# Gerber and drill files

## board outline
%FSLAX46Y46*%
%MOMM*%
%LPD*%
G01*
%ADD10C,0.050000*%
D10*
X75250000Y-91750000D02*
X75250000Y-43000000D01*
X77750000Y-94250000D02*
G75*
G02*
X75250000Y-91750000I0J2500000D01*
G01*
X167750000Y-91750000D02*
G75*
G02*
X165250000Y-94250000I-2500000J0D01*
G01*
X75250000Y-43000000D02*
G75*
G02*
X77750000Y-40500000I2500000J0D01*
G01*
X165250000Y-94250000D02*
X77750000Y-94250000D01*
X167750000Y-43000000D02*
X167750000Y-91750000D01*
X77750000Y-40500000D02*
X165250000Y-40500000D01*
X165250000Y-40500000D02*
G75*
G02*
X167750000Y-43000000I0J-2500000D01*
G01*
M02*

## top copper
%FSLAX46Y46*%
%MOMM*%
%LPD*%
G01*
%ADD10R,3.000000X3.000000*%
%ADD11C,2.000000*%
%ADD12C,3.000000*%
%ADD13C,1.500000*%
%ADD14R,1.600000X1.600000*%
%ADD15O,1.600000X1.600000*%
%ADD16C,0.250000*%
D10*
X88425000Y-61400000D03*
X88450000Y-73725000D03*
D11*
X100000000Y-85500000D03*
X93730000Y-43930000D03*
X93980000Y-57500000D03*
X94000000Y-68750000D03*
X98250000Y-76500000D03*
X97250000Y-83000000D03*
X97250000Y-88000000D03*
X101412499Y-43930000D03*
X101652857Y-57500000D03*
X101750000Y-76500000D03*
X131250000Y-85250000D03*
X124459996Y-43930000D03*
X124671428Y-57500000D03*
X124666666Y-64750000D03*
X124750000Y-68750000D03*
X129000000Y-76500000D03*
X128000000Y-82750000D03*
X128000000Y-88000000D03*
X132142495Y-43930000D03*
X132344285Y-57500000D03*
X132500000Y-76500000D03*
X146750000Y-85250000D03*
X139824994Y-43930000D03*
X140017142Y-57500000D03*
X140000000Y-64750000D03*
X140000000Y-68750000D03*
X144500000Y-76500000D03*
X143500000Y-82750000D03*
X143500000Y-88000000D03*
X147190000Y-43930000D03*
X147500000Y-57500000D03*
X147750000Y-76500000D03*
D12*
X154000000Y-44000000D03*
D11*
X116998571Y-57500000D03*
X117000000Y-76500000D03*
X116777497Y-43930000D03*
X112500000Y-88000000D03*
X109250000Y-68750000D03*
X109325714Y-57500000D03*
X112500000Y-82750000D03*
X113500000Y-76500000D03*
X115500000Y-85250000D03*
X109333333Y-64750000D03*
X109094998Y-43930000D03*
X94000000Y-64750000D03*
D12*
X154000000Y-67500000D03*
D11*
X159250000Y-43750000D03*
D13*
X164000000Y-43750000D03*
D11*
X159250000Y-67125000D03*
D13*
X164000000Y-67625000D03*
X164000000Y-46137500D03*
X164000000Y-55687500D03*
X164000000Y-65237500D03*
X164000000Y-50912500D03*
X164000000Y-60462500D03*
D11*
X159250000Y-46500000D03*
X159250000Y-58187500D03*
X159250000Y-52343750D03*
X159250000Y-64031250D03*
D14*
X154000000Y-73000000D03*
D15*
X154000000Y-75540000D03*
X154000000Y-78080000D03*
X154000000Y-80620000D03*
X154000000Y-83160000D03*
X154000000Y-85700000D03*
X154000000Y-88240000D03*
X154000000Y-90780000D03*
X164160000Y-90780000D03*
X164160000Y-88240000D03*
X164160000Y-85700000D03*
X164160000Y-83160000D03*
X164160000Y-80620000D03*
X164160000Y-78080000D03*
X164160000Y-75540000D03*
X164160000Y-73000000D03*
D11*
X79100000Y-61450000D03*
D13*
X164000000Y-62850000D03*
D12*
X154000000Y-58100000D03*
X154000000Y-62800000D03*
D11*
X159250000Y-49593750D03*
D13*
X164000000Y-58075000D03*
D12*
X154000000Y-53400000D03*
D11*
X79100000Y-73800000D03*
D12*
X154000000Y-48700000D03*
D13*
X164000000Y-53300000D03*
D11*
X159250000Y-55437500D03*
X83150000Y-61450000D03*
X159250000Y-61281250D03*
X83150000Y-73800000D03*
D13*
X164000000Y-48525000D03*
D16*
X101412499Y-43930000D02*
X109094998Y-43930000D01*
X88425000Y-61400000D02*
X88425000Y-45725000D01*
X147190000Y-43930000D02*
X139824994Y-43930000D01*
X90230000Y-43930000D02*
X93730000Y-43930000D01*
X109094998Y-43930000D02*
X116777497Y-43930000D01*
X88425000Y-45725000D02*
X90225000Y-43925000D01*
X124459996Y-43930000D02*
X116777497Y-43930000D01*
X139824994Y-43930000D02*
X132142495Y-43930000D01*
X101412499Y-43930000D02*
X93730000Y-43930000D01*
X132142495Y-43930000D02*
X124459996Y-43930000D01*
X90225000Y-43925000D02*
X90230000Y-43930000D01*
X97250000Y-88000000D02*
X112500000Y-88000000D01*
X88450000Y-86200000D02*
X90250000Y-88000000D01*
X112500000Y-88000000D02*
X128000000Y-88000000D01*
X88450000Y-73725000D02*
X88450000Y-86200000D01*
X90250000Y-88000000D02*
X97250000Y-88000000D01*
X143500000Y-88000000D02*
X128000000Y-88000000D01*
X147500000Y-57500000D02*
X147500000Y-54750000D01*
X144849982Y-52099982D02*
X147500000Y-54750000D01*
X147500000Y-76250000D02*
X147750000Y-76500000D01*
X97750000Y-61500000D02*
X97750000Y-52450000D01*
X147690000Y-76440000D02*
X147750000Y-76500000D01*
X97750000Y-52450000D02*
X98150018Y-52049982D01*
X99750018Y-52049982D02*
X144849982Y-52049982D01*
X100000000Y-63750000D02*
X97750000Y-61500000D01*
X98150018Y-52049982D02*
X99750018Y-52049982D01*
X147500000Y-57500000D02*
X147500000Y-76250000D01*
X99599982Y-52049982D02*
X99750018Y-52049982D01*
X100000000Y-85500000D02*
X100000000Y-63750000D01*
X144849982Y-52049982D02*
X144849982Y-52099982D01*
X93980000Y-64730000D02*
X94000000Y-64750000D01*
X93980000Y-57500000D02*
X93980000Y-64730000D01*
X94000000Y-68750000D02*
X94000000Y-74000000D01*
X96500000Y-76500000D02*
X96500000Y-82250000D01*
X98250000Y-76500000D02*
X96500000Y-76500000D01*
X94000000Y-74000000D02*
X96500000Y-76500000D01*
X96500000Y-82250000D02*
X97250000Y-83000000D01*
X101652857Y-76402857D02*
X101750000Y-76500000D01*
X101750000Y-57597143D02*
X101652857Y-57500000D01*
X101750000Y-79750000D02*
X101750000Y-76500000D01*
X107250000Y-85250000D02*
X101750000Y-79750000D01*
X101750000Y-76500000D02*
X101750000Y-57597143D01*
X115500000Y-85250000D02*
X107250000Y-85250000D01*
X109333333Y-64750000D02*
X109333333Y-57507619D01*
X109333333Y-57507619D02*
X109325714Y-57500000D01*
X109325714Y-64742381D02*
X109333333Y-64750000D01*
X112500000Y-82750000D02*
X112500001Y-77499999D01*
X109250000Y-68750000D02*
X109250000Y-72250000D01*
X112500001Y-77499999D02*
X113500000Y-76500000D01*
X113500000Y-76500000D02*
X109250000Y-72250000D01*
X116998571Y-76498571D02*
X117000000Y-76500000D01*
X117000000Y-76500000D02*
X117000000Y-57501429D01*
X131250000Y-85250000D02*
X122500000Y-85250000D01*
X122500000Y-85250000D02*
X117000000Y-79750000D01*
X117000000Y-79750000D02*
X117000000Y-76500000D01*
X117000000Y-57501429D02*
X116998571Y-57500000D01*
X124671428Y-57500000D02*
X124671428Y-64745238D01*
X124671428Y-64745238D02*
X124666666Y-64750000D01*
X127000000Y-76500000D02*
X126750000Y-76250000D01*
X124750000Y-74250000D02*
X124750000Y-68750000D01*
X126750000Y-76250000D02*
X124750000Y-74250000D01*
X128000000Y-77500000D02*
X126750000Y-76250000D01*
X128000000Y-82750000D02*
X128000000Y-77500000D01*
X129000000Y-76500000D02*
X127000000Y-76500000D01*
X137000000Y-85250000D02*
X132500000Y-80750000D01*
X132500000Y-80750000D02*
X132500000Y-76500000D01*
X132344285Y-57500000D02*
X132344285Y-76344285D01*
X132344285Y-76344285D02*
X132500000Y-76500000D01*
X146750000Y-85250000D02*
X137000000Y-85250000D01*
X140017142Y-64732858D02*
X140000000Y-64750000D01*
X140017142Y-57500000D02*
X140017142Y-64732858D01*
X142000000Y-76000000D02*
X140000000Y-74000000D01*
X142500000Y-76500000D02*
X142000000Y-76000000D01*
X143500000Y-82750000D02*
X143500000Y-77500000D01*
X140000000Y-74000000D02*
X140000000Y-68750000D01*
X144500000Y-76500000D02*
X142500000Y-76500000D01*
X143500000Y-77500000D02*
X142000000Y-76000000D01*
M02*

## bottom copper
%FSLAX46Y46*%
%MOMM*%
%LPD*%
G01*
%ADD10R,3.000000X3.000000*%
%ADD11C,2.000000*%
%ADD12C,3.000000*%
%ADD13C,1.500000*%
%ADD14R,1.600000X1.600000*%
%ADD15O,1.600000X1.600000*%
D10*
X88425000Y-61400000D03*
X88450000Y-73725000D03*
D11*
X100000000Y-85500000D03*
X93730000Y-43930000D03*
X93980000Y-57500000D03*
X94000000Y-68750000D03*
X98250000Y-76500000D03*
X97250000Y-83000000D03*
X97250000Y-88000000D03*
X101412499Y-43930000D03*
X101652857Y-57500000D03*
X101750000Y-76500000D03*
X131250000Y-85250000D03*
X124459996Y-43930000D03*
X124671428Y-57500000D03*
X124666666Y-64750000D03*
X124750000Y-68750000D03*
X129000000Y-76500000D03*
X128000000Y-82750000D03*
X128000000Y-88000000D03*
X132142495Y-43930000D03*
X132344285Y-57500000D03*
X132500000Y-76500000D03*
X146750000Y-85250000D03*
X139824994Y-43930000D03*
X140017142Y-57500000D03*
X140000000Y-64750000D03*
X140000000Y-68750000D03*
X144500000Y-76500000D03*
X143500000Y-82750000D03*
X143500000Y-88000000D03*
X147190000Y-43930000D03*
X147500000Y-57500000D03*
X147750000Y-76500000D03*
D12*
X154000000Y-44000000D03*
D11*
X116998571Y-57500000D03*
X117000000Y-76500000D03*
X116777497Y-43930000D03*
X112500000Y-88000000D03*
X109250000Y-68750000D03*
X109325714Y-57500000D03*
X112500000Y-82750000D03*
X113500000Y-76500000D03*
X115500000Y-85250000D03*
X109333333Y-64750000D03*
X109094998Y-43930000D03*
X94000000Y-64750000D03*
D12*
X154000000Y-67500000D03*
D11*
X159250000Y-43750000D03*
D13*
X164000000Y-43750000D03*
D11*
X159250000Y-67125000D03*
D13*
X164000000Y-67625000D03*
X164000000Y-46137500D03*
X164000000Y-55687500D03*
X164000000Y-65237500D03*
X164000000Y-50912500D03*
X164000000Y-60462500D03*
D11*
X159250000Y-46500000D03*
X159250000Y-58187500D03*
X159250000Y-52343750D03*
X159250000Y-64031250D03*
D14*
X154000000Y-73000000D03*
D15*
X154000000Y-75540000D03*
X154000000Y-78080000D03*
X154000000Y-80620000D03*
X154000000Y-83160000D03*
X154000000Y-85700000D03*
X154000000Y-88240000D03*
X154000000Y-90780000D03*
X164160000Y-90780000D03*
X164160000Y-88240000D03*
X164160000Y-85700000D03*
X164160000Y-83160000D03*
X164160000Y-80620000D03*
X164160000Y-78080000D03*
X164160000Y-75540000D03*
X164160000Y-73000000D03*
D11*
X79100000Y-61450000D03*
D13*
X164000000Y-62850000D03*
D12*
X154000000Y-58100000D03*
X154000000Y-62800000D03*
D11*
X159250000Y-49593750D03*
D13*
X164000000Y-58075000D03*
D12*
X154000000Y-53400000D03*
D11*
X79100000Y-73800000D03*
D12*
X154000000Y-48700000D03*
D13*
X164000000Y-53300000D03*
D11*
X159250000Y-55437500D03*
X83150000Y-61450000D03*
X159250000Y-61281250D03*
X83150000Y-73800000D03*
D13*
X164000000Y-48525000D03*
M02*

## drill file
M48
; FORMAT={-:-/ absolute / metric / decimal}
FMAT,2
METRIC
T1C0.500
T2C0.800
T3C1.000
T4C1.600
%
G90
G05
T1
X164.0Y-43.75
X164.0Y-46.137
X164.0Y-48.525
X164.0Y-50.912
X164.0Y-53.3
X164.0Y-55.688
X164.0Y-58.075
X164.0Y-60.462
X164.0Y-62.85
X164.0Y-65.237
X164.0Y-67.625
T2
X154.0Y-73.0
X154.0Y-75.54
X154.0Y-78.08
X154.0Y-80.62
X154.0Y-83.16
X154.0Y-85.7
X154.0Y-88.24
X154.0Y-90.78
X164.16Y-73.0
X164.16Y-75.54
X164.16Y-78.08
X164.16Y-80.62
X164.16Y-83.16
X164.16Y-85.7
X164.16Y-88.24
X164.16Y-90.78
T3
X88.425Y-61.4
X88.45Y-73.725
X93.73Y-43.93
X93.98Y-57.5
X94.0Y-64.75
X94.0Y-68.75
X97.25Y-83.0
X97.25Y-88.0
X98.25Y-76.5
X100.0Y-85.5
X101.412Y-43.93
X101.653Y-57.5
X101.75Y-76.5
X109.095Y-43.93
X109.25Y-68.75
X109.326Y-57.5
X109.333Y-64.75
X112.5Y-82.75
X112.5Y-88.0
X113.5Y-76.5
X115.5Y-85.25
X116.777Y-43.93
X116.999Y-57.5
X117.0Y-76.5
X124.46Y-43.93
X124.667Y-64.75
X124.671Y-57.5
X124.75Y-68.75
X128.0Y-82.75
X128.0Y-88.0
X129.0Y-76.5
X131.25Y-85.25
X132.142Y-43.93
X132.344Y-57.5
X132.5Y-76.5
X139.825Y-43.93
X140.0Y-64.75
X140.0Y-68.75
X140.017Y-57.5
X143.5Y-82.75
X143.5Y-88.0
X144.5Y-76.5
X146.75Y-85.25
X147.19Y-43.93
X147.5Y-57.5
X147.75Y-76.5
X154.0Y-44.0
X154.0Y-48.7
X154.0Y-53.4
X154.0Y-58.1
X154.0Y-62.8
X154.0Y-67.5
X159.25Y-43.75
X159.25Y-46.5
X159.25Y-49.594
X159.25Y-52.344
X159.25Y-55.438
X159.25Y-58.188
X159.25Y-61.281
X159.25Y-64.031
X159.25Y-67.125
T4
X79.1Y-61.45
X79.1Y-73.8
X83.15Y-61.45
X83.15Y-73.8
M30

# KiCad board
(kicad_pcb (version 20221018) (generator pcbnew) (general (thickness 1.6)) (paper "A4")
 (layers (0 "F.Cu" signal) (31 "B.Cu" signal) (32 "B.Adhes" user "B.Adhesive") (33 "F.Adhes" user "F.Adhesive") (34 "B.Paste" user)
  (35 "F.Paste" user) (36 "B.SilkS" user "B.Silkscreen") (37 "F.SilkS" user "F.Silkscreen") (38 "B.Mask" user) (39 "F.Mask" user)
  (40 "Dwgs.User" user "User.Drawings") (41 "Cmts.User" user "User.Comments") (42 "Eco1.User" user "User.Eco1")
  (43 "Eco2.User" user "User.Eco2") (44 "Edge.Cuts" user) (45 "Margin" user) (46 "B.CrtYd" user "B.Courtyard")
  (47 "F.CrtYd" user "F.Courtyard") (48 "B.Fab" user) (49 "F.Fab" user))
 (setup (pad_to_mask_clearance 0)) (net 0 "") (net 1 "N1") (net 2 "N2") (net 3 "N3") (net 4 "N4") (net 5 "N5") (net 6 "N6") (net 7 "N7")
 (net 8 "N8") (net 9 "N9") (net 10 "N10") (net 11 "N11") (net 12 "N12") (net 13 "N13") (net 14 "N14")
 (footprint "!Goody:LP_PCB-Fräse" (layer "F.Cu") (at 88.425 61.4)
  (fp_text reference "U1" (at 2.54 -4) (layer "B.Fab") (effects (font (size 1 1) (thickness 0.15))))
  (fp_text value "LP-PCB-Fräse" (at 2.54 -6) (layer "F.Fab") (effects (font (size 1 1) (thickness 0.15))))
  (pad "1" thru_hole rect (at 0 0) (size 3 3) (drill 1) (layers "*.Cu" "*.Mask") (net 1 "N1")))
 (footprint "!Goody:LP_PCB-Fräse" (layer "F.Cu") (at 88.45 73.725)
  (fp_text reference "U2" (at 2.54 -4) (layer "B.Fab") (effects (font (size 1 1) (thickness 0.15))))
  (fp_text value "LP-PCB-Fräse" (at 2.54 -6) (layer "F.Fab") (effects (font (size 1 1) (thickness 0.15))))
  (pad "1" thru_hole rect (at 0 0) (size 3 3) (drill 1) (layers "*.Cu" "*.Mask") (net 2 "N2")))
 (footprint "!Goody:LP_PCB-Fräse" (layer "F.Cu") (at 100 85.5)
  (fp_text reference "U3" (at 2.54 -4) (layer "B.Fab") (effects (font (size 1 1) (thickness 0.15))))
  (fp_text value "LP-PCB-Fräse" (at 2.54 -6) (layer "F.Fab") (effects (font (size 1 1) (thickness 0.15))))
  (pad "1" thru_hole circle (at 0 0) (size 2 2) (drill 1) (layers "*.Cu" "*.Mask") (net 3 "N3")))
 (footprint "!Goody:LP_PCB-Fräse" (layer "F.Cu") (at 93.73 43.93)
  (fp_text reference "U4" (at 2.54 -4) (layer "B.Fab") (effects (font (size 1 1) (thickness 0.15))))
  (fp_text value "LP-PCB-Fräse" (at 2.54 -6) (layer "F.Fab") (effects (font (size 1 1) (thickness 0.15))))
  (pad "1" thru_hole circle (at 0 0) (size 2 2) (drill 1) (layers "*.Cu" "*.Mask") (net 1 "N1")))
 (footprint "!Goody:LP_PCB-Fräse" (layer "F.Cu") (at 93.98 57.5)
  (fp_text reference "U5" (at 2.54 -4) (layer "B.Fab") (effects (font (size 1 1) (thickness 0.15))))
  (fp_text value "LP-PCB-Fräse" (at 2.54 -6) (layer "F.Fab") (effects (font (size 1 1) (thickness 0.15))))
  (pad "1" thru_hole circle (at 0 0) (size 2 2) (drill 1) (layers "*.Cu" "*.Mask") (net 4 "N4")))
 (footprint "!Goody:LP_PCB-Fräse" (layer "F.Cu") (at 94 68.75)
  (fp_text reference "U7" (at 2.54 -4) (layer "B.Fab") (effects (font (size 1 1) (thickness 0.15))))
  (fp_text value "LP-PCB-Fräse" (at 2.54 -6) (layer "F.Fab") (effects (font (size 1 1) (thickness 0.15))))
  (pad "1" thru_hole circle (at 0 0) (size 2 2) (drill 1) (layers "*.Cu" "*.Mask") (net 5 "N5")))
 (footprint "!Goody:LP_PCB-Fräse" (layer "F.Cu") (at 98.25 76.5)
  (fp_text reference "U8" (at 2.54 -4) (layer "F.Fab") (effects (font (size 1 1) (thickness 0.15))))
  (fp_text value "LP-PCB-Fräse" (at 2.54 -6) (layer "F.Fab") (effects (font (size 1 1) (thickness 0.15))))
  (pad "1" thru_hole circle (at 0 0) (size 2 2) (drill 1) (layers "*.Cu" "*.Mask") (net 5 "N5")))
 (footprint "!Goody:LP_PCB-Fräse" (layer "F.Cu") (at 97.25 83)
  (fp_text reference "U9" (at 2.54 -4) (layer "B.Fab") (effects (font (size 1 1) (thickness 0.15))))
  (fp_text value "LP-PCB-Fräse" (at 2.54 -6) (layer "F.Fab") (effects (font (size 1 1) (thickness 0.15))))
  (pad "1" thru_hole circle (at 0 0) (size 2 2) (drill 1) (layers "*.Cu" "*.Mask") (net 5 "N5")))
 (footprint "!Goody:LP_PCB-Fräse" (layer "F.Cu") (at 97.25 88)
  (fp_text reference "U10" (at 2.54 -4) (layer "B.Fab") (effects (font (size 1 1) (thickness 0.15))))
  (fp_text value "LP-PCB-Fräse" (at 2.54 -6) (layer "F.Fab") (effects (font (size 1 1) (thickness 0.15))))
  (pad "1" thru_hole circle (at 0 0) (size 2 2) (drill 1) (layers "*.Cu" "*.Mask") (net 2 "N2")))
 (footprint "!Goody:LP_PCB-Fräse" (layer "F.Cu") (at 101.412499 43.93)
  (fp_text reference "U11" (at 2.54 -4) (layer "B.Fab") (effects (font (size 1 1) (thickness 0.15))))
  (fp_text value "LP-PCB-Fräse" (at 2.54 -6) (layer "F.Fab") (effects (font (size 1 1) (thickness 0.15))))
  (pad "1" thru_hole circle (at 0 0) (size 2 2) (drill 1) (layers "*.Cu" "*.Mask") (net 1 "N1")))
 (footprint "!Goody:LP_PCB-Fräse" (layer "F.Cu") (at 101.652857 57.5)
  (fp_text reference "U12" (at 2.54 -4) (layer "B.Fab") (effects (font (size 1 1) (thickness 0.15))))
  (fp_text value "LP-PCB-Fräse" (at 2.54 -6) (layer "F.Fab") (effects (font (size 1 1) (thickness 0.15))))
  (pad "1" thru_hole circle (at 0 0) (size 2 2) (drill 1) (layers "*.Cu" "*.Mask") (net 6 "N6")))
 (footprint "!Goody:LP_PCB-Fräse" (layer "F.Cu") (at 101.75 76.5)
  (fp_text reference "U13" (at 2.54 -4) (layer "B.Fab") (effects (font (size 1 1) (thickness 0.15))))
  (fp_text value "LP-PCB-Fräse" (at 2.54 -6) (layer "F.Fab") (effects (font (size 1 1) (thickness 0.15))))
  (pad "1" thru_hole circle (at 0 0) (size 2 2) (drill 1) (layers "*.Cu" "*.Mask") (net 6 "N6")))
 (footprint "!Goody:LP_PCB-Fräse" (layer "F.Cu") (at 131.25 85.25)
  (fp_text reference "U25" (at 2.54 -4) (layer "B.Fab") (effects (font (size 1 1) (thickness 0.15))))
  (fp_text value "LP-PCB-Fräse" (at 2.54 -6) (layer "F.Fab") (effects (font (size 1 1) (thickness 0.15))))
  (pad "1" thru_hole circle (at 0 0) (size 2 2) (drill 1) (layers "*.Cu" "*.Mask") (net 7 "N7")))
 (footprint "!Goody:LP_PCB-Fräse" (layer "F.Cu") (at 124.459996 43.93)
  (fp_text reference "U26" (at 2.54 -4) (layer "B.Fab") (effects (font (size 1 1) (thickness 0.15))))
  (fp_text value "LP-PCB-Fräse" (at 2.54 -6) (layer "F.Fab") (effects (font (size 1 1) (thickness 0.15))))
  (pad "1" thru_hole circle (at 0 0) (size 2 2) (drill 1) (layers "*.Cu" "*.Mask") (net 1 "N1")))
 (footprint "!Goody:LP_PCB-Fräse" (layer "F.Cu") (at 124.671428 57.5)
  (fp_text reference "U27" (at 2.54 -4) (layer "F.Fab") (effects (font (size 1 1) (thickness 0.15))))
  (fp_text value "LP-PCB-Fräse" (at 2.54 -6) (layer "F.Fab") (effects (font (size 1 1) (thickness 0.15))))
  (pad "1" thru_hole circle (at 0 0) (size 2 2) (drill 1) (layers "*.Cu" "*.Mask") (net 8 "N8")))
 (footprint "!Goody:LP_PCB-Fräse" (layer "F.Cu") (at 124.666666 64.75)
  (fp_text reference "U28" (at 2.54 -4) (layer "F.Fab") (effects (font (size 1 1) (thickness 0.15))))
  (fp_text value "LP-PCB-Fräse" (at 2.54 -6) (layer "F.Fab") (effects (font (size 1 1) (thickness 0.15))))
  (pad "1" thru_hole circle (at 0 0) (size 2 2) (drill 1) (layers "*.Cu" "*.Mask") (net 8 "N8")))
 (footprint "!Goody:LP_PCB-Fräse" (layer "F.Cu") (at 124.75 68.75)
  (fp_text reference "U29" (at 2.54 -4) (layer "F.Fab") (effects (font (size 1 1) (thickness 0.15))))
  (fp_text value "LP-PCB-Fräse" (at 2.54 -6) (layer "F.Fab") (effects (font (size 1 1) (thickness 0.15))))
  (pad "1" thru_hole circle (at 0 0) (size 2 2) (drill 1) (layers "*.Cu" "*.Mask") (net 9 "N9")))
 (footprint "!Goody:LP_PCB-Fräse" (layer "F.Cu") (at 129 76.5)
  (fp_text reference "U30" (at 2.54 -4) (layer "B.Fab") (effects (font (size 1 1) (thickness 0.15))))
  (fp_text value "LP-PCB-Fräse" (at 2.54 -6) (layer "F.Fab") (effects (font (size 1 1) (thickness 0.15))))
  (pad "1" thru_hole circle (at 0 0) (size 2 2) (drill 1) (layers "*.Cu" "*.Mask") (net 9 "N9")))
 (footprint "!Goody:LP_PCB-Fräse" (layer "F.Cu") (at 128 82.75)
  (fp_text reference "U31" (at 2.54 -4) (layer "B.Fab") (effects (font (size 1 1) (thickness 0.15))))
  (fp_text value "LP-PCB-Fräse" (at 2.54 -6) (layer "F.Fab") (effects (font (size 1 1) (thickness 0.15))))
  (pad "1" thru_hole circle (at 0 0) (size 2 2) (drill 1) (layers "*.Cu" "*.Mask") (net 9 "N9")))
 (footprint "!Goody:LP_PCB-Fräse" (layer "F.Cu") (at 128 88)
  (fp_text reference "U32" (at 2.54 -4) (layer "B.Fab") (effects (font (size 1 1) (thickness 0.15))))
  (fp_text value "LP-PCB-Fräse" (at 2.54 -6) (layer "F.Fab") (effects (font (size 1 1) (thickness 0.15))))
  (pad "1" thru_hole circle (at 0 0) (size 2 2) (drill 1) (layers "*.Cu" "*.Mask") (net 2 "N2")))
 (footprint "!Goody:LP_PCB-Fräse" (layer "F.Cu") (at 132.142495 43.93)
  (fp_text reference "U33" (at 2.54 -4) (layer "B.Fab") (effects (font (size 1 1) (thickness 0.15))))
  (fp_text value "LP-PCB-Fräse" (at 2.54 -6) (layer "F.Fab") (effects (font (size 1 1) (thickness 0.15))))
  (pad "1" thru_hole circle (at 0 0) (size 2 2) (drill 1) (layers "*.Cu" "*.Mask") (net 1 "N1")))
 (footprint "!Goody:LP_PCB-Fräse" (layer "F.Cu") (at 132.344285 57.5)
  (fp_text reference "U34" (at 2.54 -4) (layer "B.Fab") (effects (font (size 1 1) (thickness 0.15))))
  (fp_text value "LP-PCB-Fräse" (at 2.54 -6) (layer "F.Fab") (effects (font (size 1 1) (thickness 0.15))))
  (pad "1" thru_hole circle (at 0 0) (size 2 2) (drill 1) (layers "*.Cu" "*.Mask") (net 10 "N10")))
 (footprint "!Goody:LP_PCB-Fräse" (layer "F.Cu") (at 132.5 76.5)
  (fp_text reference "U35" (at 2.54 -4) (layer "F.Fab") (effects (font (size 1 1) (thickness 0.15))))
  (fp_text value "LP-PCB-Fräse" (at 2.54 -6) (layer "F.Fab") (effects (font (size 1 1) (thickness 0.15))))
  (pad "1" thru_hole circle (at 0 0) (size 2 2) (drill 1) (layers "*.Cu" "*.Mask") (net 10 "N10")))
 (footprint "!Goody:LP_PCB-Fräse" (layer "F.Cu") (at 146.75 85.25)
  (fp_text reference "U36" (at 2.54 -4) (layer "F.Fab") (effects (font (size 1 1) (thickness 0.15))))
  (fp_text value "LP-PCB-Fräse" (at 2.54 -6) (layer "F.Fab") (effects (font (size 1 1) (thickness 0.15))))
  (pad "1" thru_hole circle (at 0 0) (size 2 2) (drill 1) (layers "*.Cu" "*.Mask") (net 10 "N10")))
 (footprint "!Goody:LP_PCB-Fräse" (layer "F.Cu") (at 139.824994 43.93)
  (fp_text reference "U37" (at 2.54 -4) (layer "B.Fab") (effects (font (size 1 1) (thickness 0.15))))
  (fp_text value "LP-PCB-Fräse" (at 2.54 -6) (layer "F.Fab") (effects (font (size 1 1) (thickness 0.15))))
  (pad "1" thru_hole circle (at 0 0) (size 2 2) (drill 1) (layers "*.Cu" "*.Mask") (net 1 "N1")))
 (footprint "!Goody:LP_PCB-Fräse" (layer "F.Cu") (at 140.017142 57.5)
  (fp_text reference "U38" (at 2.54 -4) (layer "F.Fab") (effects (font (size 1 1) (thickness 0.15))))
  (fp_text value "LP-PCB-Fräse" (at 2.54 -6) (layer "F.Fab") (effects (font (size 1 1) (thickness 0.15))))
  (pad "1" thru_hole circle (at 0 0) (size 2 2) (drill 1) (layers "*.Cu" "*.Mask") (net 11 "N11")))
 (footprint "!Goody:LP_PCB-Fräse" (layer "F.Cu") (at 140 64.75)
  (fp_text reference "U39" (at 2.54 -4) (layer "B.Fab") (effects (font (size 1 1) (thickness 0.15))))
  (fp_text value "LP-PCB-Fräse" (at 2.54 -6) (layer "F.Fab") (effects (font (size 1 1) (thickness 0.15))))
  (pad "1" thru_hole circle (at 0 0) (size 2 2) (drill 1) (layers "*.Cu" "*.Mask") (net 11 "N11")))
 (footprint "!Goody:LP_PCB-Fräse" (layer "F.Cu") (at 140 68.75)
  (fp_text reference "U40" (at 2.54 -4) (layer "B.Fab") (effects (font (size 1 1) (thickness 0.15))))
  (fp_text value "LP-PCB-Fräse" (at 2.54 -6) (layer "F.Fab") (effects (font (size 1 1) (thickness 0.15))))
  (pad "1" thru_hole circle (at 0 0) (size 2 2) (drill 1) (layers "*.Cu" "*.Mask") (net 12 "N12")))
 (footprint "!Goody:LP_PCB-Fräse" (layer "F.Cu") (at 144.5 76.5)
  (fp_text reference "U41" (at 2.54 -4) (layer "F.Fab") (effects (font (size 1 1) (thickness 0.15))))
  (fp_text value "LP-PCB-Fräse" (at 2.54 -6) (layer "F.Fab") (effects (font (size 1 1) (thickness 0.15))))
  (pad "1" thru_hole circle (at 0 0) (size 2 2) (drill 1) (layers "*.Cu" "*.Mask") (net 12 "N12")))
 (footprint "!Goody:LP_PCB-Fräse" (layer "F.Cu") (at 143.5 82.75)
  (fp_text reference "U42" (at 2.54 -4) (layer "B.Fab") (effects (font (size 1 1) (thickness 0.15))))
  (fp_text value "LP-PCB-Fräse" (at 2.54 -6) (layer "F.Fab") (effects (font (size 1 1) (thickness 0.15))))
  (pad "1" thru_hole circle (at 0 0) (size 2 2) (drill 1) (layers "*.Cu" "*.Mask") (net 12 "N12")))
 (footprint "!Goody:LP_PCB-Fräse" (layer "F.Cu") (at 143.5 88)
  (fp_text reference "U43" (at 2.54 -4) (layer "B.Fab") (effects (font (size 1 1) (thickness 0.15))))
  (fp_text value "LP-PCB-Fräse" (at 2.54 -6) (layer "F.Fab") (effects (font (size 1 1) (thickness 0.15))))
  (pad "1" thru_hole circle (at 0 0) (size 2 2) (drill 1) (layers "*.Cu" "*.Mask") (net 2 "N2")))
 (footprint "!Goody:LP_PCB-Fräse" (layer "F.Cu") (at 147.19 43.93)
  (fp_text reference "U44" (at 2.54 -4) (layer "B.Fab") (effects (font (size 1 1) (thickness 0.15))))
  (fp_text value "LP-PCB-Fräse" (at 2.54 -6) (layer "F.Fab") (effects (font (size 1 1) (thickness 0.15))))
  (pad "1" thru_hole circle (at 0 0) (size 2 2) (drill 1) (layers "*.Cu" "*.Mask") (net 1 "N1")))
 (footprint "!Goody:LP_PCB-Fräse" (layer "F.Cu") (at 147.5 57.5)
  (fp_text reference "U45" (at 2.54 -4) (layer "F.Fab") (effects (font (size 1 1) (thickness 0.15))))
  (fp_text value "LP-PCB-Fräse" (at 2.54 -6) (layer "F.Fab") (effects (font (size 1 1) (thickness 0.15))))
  (pad "1" thru_hole circle (at 0 0) (size 2 2) (drill 1) (layers "*.Cu" "*.Mask") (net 3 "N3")))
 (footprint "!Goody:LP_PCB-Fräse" (layer "F.Cu") (at 147.75 76.5)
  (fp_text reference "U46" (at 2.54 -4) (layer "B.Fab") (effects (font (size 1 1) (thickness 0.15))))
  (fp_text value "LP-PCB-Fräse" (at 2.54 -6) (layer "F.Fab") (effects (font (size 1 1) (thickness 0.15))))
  (pad "1" thru_hole circle (at 0 0) (size 2 2) (drill 1) (layers "*.Cu" "*.Mask") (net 3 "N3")))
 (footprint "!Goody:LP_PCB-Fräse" (layer "F.Cu") (at 154 44)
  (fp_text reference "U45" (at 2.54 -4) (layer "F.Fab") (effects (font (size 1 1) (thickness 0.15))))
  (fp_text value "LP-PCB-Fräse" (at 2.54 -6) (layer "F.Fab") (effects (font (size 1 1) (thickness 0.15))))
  (pad "1" thru_hole circle (at 0 0) (size 3 3) (drill 1) (layers "*.Cu" "*.Mask")))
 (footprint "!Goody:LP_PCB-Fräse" (layer "F.Cu") (at 116.998571 57.5)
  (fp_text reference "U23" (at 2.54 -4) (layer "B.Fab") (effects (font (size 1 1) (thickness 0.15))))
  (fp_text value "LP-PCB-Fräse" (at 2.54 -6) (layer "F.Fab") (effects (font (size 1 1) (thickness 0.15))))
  (pad "1" thru_hole circle (at 0 0) (size 2 2) (drill 1) (layers "*.Cu" "*.Mask") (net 7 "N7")))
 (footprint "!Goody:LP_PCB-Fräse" (layer "F.Cu") (at 117 76.5)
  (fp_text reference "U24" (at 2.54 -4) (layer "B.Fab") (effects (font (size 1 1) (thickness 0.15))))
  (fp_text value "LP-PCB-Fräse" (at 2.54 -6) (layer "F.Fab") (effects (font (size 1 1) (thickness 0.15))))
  (pad "1" thru_hole circle (at 0 0) (size 2 2) (drill 1) (layers "*.Cu" "*.Mask") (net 7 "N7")))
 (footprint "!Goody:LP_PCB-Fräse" (layer "F.Cu") (at 116.777497 43.93)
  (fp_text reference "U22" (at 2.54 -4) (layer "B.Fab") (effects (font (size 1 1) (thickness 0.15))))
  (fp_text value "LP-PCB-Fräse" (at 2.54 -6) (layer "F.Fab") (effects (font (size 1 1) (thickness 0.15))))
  (pad "1" thru_hole circle (at 0 0) (size 2 2) (drill 1) (layers "*.Cu" "*.Mask") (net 1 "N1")))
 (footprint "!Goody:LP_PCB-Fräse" (layer "F.Cu") (at 112.5 88)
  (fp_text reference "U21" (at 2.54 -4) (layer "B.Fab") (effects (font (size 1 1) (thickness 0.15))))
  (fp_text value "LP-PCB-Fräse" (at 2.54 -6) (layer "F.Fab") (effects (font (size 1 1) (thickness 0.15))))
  (pad "1" thru_hole circle (at 0 0) (size 2 2) (drill 1) (layers "*.Cu" "*.Mask") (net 2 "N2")))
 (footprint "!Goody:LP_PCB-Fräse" (layer "F.Cu") (at 109.25 68.75)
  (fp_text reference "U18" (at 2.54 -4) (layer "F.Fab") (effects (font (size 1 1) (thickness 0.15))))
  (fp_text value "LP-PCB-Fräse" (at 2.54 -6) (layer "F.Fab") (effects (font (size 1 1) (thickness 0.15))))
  (pad "1" thru_hole circle (at 0 0) (size 2 2) (drill 1) (layers "*.Cu" "*.Mask") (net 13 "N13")))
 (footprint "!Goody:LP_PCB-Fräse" (layer "F.Cu") (at 109.325714 57.5)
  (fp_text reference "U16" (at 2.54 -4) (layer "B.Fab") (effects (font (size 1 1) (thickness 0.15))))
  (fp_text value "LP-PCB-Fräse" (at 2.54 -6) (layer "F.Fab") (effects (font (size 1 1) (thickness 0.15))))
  (pad "1" thru_hole circle (at 0 0) (size 2 2) (drill 1) (layers "*.Cu" "*.Mask") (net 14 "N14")))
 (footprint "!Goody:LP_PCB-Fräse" (layer "F.Cu") (at 112.5 82.75)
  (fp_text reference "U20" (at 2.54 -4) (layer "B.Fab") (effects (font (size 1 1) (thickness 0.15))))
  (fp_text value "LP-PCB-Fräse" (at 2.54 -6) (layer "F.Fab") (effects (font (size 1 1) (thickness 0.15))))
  (pad "1" thru_hole circle (at 0 0) (size 2 2) (drill 1) (layers "*.Cu" "*.Mask") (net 13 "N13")))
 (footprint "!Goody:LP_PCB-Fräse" (layer "F.Cu") (at 113.5 76.5)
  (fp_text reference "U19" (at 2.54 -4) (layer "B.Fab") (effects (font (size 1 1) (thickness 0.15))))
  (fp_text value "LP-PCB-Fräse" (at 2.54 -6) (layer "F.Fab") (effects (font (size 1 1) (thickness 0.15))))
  (pad "1" thru_hole circle (at 0 0) (size 2 2) (drill 1) (layers "*.Cu" "*.Mask") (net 13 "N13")))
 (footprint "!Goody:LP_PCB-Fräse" (layer "F.Cu") (at 115.5 85.25)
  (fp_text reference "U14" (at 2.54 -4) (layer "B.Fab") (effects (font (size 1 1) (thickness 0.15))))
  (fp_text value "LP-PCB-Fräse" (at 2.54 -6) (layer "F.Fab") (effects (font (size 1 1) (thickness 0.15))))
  (pad "1" thru_hole circle (at 0 0) (size 2 2) (drill 1) (layers "*.Cu" "*.Mask") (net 6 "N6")))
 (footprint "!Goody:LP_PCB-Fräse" (layer "F.Cu") (at 109.333333 64.75)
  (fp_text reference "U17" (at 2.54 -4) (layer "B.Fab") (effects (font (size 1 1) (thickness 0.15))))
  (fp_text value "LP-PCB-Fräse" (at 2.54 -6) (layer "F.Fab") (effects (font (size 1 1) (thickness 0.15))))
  (pad "" thru_hole circle (at 0 0) (size 2 2) (drill 1) (layers "*.Cu" "*.Mask") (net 14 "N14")))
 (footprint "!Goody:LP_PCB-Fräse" (layer "F.Cu") (at 109.094998 43.93)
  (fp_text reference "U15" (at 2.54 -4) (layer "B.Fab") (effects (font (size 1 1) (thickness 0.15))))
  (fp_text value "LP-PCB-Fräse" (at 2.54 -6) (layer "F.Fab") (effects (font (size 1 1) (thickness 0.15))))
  (pad "1" thru_hole circle (at 0 0) (size 2 2) (drill 1) (layers "*.Cu" "*.Mask") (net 1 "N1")))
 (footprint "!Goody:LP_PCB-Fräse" (layer "F.Cu") (at 94 64.75)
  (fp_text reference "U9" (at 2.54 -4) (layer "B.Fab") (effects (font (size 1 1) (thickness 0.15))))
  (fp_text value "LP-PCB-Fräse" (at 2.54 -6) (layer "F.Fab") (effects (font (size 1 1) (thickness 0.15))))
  (pad "1" thru_hole circle (at 0 0) (size 2 2) (drill 1) (layers "*.Cu" "*.Mask") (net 4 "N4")))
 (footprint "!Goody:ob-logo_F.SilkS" (layer "F.Cu") (at 85.925 83.125)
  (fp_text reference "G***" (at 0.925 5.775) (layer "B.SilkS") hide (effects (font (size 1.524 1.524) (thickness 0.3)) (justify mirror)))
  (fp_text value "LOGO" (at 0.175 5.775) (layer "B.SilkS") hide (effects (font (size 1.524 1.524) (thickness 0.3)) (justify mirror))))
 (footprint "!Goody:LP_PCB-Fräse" (layer "F.Cu") (at 154 67.5)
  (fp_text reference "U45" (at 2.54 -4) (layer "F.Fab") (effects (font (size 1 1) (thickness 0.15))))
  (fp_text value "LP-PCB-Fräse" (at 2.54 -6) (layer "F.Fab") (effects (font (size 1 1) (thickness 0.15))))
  (pad "1" thru_hole circle (at 0 0) (size 3 3) (drill 1) (layers "*.Cu" "*.Mask")))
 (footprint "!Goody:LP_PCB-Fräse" (layer "F.Cu") (at 159.25 43.75)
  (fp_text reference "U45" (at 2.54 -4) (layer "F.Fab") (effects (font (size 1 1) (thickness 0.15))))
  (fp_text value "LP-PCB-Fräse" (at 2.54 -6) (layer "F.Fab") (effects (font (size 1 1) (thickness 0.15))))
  (pad "1" thru_hole circle (at 0 0) (size 2 2) (drill 1) (layers "*.Cu" "*.Mask")))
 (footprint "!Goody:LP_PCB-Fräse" (layer "F.Cu") (at 164 43.75)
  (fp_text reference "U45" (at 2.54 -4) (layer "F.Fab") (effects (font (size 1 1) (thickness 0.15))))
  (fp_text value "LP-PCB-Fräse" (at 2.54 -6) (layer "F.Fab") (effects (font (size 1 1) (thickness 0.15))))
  (pad "1" thru_hole circle (at 0 0) (size 1.5 1.5) (drill 0.5) (layers "*.Cu" "*.Mask")))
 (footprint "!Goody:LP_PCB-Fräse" (layer "F.Cu") (at 159.25 67.125)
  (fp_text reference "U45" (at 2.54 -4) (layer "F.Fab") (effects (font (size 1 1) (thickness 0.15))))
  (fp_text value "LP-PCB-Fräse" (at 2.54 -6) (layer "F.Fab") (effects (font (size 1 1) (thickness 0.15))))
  (pad "1" thru_hole circle (at 0 0) (size 2 2) (drill 1) (layers "*.Cu" "*.Mask")))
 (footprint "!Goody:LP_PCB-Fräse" (layer "F.Cu") (at 164 67.625)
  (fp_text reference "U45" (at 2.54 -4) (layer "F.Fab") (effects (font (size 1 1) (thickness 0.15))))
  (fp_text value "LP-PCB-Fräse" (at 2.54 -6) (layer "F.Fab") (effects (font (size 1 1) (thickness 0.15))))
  (pad "1" thru_hole circle (at 0 0) (size 1.5 1.5) (drill 0.5) (layers "*.Cu" "*.Mask")))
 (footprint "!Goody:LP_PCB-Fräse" (layer "F.Cu") (at 164 46.1375)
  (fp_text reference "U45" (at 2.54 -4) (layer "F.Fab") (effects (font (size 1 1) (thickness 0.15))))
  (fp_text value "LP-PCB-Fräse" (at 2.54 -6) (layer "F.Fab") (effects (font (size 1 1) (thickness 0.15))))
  (pad "1" thru_hole circle (at 0 0) (size 1.5 1.5) (drill 0.5) (layers "*.Cu" "*.Mask")))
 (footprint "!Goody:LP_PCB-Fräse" (layer "F.Cu") (at 164 55.6875)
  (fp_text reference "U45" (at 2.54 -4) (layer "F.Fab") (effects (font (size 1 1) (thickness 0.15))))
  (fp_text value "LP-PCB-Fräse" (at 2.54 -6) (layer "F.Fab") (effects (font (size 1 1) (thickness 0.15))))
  (pad "1" thru_hole circle (at 0 0) (size 1.5 1.5) (drill 0.5) (layers "*.Cu" "*.Mask")))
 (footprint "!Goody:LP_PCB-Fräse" (layer "F.Cu") (at 164 65.2375)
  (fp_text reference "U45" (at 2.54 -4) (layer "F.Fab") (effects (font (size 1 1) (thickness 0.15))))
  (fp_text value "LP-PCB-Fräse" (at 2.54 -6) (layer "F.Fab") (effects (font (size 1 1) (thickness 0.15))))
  (pad "1" thru_hole circle (at 0 0) (size 1.5 1.5) (drill 0.5) (layers "*.Cu" "*.Mask")))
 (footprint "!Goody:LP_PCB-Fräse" (layer "F.Cu") (at 164 50.9125)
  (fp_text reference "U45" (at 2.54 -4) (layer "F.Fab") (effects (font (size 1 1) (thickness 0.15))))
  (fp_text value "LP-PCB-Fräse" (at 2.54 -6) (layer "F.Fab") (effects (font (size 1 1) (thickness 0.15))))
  (pad "1" thru_hole circle (at 0 0) (size 1.5 1.5) (drill 0.5) (layers "*.Cu" "*.Mask")))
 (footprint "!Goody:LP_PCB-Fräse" (layer "F.Cu") (at 164 60.4625)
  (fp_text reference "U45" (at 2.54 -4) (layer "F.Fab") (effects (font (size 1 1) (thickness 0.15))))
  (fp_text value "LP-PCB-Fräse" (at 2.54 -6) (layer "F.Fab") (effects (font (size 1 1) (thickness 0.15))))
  (pad "1" thru_hole circle (at 0 0) (size 1.5 1.5) (drill 0.5) (layers "*.Cu" "*.Mask")))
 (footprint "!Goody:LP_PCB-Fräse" (layer "F.Cu") (at 159.25 46.5)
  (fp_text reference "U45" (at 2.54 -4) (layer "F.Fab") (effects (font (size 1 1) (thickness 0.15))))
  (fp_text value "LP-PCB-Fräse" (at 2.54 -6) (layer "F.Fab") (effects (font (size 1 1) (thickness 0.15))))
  (pad "1" thru_hole circle (at 0 0) (size 2 2) (drill 1) (layers "*.Cu" "*.Mask")))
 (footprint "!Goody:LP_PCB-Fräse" (layer "F.Cu") (at 159.25 58.1875)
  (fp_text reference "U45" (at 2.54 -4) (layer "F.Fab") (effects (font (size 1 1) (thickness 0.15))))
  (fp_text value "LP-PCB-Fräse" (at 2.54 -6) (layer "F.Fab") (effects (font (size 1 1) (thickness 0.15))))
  (pad "1" thru_hole circle (at 0 0) (size 2 2) (drill 1) (layers "*.Cu" "*.Mask")))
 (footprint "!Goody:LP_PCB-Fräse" (layer "F.Cu") (at 159.25 52.34375)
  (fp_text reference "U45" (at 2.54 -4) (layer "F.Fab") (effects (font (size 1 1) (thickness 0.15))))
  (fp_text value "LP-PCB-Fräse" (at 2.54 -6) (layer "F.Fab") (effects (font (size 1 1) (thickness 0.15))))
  (pad "1" thru_hole circle (at 0 0) (size 2 2) (drill 1) (layers "*.Cu" "*.Mask")))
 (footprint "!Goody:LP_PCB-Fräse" (layer "F.Cu") (at 159.25 64.03125)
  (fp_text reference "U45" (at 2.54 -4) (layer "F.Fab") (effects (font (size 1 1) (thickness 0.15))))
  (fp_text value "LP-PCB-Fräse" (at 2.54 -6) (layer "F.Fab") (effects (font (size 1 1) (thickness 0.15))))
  (pad "1" thru_hole circle (at 0 0) (size 2 2) (drill 1) (layers "*.Cu" "*.Mask")))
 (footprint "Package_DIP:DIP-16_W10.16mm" (layer "F.Cu") (at 154 73)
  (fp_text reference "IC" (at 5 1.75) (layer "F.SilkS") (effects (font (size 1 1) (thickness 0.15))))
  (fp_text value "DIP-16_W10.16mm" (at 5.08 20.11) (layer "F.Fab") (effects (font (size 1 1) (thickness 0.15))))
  (pad "1" thru_hole rect (at 0 0) (size 1.6 1.6) (drill 0.8) (layers "*.Cu" "*.Mask"))
  (pad "2" thru_hole oval (at 0 2.54) (size 1.6 1.6) (drill 0.8) (layers "*.Cu" "*.Mask"))
  (pad "3" thru_hole oval (at 0 5.08) (size 1.6 1.6) (drill 0.8) (layers "*.Cu" "*.Mask"))
  (pad "4" thru_hole oval (at 0 7.62) (size 1.6 1.6) (drill 0.8) (layers "*.Cu" "*.Mask"))
  (pad "5" thru_hole oval (at 0 10.16) (size 1.6 1.6) (drill 0.8) (layers "*.Cu" "*.Mask"))
  (pad "6" thru_hole oval (at 0 12.7) (size 1.6 1.6) (drill 0.8) (layers "*.Cu" "*.Mask"))
  (pad "7" thru_hole oval (at 0 15.24) (size 1.6 1.6) (drill 0.8) (layers "*.Cu" "*.Mask"))
  (pad "8" thru_hole oval (at 0 17.78) (size 1.6 1.6) (drill 0.8) (layers "*.Cu" "*.Mask"))
  (pad "9" thru_hole oval (at 10.16 17.78) (size 1.6 1.6) (drill 0.8) (layers "*.Cu" "*.Mask"))
  (pad "10" thru_hole oval (at 10.16 15.24) (size 1.6 1.6) (drill 0.8) (layers "*.Cu" "*.Mask"))
  (pad "11" thru_hole oval (at 10.16 12.7) (size 1.6 1.6) (drill 0.8) (layers "*.Cu" "*.Mask"))
  (pad "12" thru_hole oval (at 10.16 10.16) (size 1.6 1.6) (drill 0.8) (layers "*.Cu" "*.Mask"))
  (pad "13" thru_hole oval (at 10.16 7.62) (size 1.6 1.6) (drill 0.8) (layers "*.Cu" "*.Mask"))
  (pad "14" thru_hole oval (at 10.16 5.08) (size 1.6 1.6) (drill 0.8) (layers "*.Cu" "*.Mask"))
  (pad "15" thru_hole oval (at 10.16 2.54) (size 1.6 1.6) (drill 0.8) (layers "*.Cu" "*.Mask"))
  (pad "16" thru_hole oval (at 10.16 0) (size 1.6 1.6) (drill 0.8) (layers "*.Cu" "*.Mask")))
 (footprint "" (layer "F.Cu") (at 79.1 61.45)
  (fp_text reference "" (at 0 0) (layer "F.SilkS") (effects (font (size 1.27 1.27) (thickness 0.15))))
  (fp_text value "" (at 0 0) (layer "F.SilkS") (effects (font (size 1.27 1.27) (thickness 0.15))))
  (pad "" thru_hole circle (at 0 0) (size 2 2) (drill 1.6) (layers "*.Cu" "*.Mask")))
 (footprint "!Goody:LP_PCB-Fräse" (layer "F.Cu") (at 164 62.85)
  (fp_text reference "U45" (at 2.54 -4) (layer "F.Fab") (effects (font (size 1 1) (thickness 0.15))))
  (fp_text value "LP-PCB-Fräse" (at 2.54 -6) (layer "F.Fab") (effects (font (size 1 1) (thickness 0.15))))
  (pad "1" thru_hole circle (at 0 0) (size 1.5 1.5) (drill 0.5) (layers "*.Cu" "*.Mask")))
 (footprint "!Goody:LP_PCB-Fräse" (layer "F.Cu") (at 154 58.1)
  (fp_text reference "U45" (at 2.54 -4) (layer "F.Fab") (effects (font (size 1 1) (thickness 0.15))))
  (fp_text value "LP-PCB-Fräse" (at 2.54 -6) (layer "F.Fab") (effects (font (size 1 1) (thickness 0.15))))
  (pad "1" thru_hole circle (at 0 0) (size 3 3) (drill 1) (layers "*.Cu" "*.Mask")))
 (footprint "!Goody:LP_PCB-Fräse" (layer "F.Cu") (at 154 62.8)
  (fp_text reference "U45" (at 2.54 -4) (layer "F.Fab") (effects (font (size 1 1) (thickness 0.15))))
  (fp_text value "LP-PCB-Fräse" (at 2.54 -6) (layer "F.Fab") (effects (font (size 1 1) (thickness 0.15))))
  (pad "1" thru_hole circle (at 0 0) (size 3 3) (drill 1) (layers "*.Cu" "*.Mask")))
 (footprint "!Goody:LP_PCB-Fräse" (layer "F.Cu") (at 159.25 49.59375)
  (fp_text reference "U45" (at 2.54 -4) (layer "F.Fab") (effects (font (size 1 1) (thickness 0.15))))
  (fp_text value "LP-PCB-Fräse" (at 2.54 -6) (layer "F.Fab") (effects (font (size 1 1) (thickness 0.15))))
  (pad "1" thru_hole circle (at 0 0) (size 2 2) (drill 1) (layers "*.Cu" "*.Mask")))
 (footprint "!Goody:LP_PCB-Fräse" (layer "F.Cu") (at 164 58.075)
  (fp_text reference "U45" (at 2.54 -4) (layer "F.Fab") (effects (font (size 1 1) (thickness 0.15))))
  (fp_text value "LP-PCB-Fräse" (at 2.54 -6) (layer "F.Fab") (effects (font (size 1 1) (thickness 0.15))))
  (pad "1" thru_hole circle (at 0 0) (size 1.5 1.5) (drill 0.5) (layers "*.Cu" "*.Mask")))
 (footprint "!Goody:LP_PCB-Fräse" (layer "F.Cu") (at 154 53.4)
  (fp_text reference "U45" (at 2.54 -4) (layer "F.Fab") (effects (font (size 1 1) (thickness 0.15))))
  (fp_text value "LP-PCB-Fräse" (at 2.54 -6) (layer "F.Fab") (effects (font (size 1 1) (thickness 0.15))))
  (pad "1" thru_hole circle (at 0 0) (size 3 3) (drill 1) (layers "*.Cu" "*.Mask")))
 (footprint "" (layer "F.Cu") (at 79.1 73.8)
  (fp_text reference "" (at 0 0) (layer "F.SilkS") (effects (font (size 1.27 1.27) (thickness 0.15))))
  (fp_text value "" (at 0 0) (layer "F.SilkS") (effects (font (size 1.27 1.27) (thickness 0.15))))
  (pad "" thru_hole circle (at 0 0) (size 2 2) (drill 1.6) (layers "*.Cu" "*.Mask")))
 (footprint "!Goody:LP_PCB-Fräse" (layer "F.Cu") (at 154 48.7)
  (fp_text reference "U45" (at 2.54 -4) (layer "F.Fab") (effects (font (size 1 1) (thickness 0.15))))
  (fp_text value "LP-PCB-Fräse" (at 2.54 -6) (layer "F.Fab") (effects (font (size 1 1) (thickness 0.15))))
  (pad "1" thru_hole circle (at 0 0) (size 3 3) (drill 1) (layers "*.Cu" "*.Mask")))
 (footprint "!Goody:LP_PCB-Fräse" (layer "F.Cu") (at 164 53.3)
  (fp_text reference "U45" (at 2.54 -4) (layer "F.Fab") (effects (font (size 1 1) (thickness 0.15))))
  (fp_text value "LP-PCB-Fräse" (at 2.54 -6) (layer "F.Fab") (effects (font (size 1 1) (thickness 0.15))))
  (pad "1" thru_hole circle (at 0 0) (size 1.5 1.5) (drill 0.5) (layers "*.Cu" "*.Mask")))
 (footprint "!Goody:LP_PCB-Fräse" (layer "F.Cu") (at 159.25 55.4375)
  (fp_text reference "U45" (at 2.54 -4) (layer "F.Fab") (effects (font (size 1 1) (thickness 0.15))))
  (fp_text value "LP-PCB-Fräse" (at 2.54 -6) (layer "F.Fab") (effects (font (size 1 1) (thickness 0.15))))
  (pad "1" thru_hole circle (at 0 0) (size 2 2) (drill 1) (layers "*.Cu" "*.Mask")))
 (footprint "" (layer "F.Cu") (at 83.15 61.45)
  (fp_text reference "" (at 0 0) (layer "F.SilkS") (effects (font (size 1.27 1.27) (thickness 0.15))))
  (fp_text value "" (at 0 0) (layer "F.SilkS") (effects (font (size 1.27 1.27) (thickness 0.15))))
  (pad "" thru_hole circle (at 0 0) (size 2 2) (drill 1.6) (layers "*.Cu" "*.Mask")))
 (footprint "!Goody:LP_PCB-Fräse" (layer "F.Cu") (at 159.25 61.28125)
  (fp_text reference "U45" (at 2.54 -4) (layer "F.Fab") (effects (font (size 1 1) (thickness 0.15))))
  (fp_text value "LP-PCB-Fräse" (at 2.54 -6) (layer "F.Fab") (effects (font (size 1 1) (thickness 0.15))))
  (pad "1" thru_hole circle (at 0 0) (size 2 2) (drill 1) (layers "*.Cu" "*.Mask")))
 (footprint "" (layer "F.Cu") (at 83.15 73.8)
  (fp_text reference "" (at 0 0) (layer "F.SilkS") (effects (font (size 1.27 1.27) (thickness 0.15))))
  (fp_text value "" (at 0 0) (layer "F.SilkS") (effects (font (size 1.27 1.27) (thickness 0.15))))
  (pad "" thru_hole circle (at 0 0) (size 2 2) (drill 1.6) (layers "*.Cu" "*.Mask")))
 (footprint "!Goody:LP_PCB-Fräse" (layer "F.Cu") (at 164 48.525)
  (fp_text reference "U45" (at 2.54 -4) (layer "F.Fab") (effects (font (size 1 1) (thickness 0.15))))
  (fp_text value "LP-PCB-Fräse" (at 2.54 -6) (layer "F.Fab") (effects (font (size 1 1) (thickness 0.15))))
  (pad "1" thru_hole circle (at 0 0) (size 1.5 1.5) (drill 0.5) (layers "*.Cu" "*.Mask")))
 (gr_line (start 75.25 91.75) (end 75.25 43) (stroke (width 0.05) (type solid)) (layer "Edge.Cuts"))
 (gr_arc (start 77.75 94.25) (mid 75.982233 93.517767) (end 75.25 91.75) (stroke (width 0.05) (type solid)) (layer "Edge.Cuts"))
 (gr_arc (start 167.75 91.75) (mid 167.017767 93.517767) (end 165.25 94.25) (stroke (width 0.05) (type solid)) (layer "Edge.Cuts"))
 (gr_arc (start 75.25 43) (mid 75.982233 41.232233) (end 77.75 40.5) (stroke (width 0.05) (type solid)) (layer "Edge.Cuts"))
 (gr_line (start 165.25 94.25) (end 77.75 94.25) (stroke (width 0.05) (type solid)) (layer "Edge.Cuts"))
 (gr_line (start 167.75 43) (end 167.75 91.75) (stroke (width 0.05) (type solid)) (layer "Edge.Cuts"))
 (gr_line (start 77.75 40.5) (end 165.25 40.5) (stroke (width 0.05) (type solid)) (layer "Edge.Cuts"))
 (gr_arc (start 165.25 40.5) (mid 167.017767 41.232233) (end 167.75 43) (stroke (width 0.05) (type solid)) (layer "Edge.Cuts"))
 (segment (start 101.412499 43.93) (end 109.094998 43.93) (width 0.25) (layer "F.Cu") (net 1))
 (segment (start 88.425 61.4) (end 88.425 45.725) (width 0.25) (layer "F.Cu") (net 1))
 (segment (start 147.19 43.93) (end 139.824994 43.93) (width 0.25) (layer "F.Cu") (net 1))
 (segment (start 90.23 43.93) (end 93.73 43.93) (width 0.25) (layer "F.Cu") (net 1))
 (segment (start 109.094998 43.93) (end 116.777497 43.93) (width 0.25) (layer "F.Cu") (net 1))
 (segment (start 88.425 45.725) (end 90.225 43.925) (width 0.25) (layer "F.Cu") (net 1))
 (segment (start 124.459996 43.93) (end 116.777497 43.93) (width 0.25) (layer "F.Cu") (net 1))
 (segment (start 139.824994 43.93) (end 132.142495 43.93) (width 0.25) (layer "F.Cu") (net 1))
 (segment (start 101.412499 43.93) (end 93.73 43.93) (width 0.25) (layer "F.Cu") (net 1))
 (segment (start 132.142495 43.93) (end 124.459996 43.93) (width 0.25) (layer "F.Cu") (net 1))
 (segment (start 90.225 43.925) (end 90.23 43.93) (width 0.25) (layer "F.Cu") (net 1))
 (segment (start 97.25 88) (end 112.5 88) (width 0.25) (layer "F.Cu") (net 2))
 (segment (start 88.45 86.2) (end 90.25 88) (width 0.25) (layer "F.Cu") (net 2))
 (segment (start 112.5 88) (end 128 88) (width 0.25) (layer "F.Cu") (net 2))
 (segment (start 88.45 73.725) (end 88.45 86.2) (width 0.25) (layer "F.Cu") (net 2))
 (segment (start 90.25 88) (end 97.25 88) (width 0.25) (layer "F.Cu") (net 2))
 (segment (start 143.5 88) (end 128 88) (width 0.25) (layer "F.Cu") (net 2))
 (segment (start 147.5 57.5) (end 147.5 54.75) (width 0.25) (layer "F.Cu") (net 3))
 (segment (start 144.849982 52.099982) (end 147.5 54.75) (width 0.25) (layer "F.Cu") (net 3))
 (segment (start 147.5 76.25) (end 147.75 76.5) (width 0.25) (layer "F.Cu") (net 3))
 (segment (start 97.75 61.5) (end 97.75 52.45) (width 0.25) (layer "F.Cu") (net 3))
 (segment (start 147.69 76.44) (end 147.75 76.5) (width 0.25) (layer "F.Cu") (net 3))
 (segment (start 97.75 52.45) (end 98.150018 52.049982) (width 0.25) (layer "F.Cu") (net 3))
 (segment (start 99.750018 52.049982) (end 144.849982 52.049982) (width 0.25) (layer "F.Cu") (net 3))
 (segment (start 100 63.75) (end 97.75 61.5) (width 0.25) (layer "F.Cu") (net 3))
 (segment (start 98.150018 52.049982) (end 99.750018 52.049982) (width 0.25) (layer "F.Cu") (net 3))
 (segment (start 147.5 57.5) (end 147.5 76.25) (width 0.25) (layer "F.Cu") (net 3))
 (segment (start 99.599982 52.049982) (end 99.750018 52.049982) (width 0.25) (layer "F.Cu") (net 3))
 (segment (start 100 85.5) (end 100 63.75) (width 0.25) (layer "F.Cu") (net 3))
 (segment (start 144.849982 52.049982) (end 144.849982 52.099982) (width 0.25) (layer "F.Cu") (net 3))
 (segment (start 93.98 64.73) (end 94 64.75) (width 0.25) (layer "F.Cu") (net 4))
 (segment (start 93.98 57.5) (end 93.98 64.73) (width 0.25) (layer "F.Cu") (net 4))
 (segment (start 94 68.75) (end 94 74) (width 0.25) (layer "F.Cu") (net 5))
 (segment (start 96.5 76.5) (end 96.5 82.25) (width 0.25) (layer "F.Cu") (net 5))
 (segment (start 98.25 76.5) (end 96.5 76.5) (width 0.25) (layer "F.Cu") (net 5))
 (segment (start 94 74) (end 96.5 76.5) (width 0.25) (layer "F.Cu") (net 5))
 (segment (start 96.5 82.25) (end 97.25 83) (width 0.25) (layer "F.Cu") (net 5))
 (segment (start 101.652857 76.402857) (end 101.75 76.5) (width 0.25) (layer "F.Cu") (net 6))
 (segment (start 101.75 57.597143) (end 101.652857 57.5) (width 0.25) (layer "F.Cu") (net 6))
 (segment (start 101.75 79.75) (end 101.75 76.5) (width 0.25) (layer "F.Cu") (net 6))
 (segment (start 107.25 85.25) (end 101.75 79.75) (width 0.25) (layer "F.Cu") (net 6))
 (segment (start 101.75 76.5) (end 101.75 57.597143) (width 0.25) (layer "F.Cu") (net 6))
 (segment (start 115.5 85.25) (end 107.25 85.25) (width 0.25) (layer "F.Cu") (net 6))
 (segment (start 109.333333 64.75) (end 109.333333 57.507619) (width 0.25) (layer "F.Cu") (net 14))
 (segment (start 109.333333 57.507619) (end 109.325714 57.5) (width 0.25) (layer "F.Cu") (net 14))
 (segment (start 109.325714 64.742381) (end 109.333333 64.75) (width 0.25) (layer "F.Cu") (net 14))
 (segment (start 112.5 82.75) (end 112.500001 77.499999) (width 0.25) (layer "F.Cu") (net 13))
 (segment (start 109.25 68.75) (end 109.25 72.25) (width 0.25) (layer "F.Cu") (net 13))
 (segment (start 112.500001 77.499999) (end 113.5 76.5) (width 0.25) (layer "F.Cu") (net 13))
 (segment (start 113.5 76.5) (end 109.25 72.25) (width 0.25) (layer "F.Cu") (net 13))
 (segment (start 116.998571 76.498571) (end 117 76.5) (width 0.25) (layer "F.Cu") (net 7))
 (segment (start 117 76.5) (end 117 57.501429) (width 0.25) (layer "F.Cu") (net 7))
 (segment (start 131.25 85.25) (end 122.5 85.25) (width 0.25) (layer "F.Cu") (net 7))
 (segment (start 122.5 85.25) (end 117 79.75) (width 0.25) (layer "F.Cu") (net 7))
 (segment (start 117 79.75) (end 117 76.5) (width 0.25) (layer "F.Cu") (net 7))
 (segment (start 117 57.501429) (end 116.998571 57.5) (width 0.25) (layer "F.Cu") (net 7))
 (segment (start 124.671428 57.5) (end 124.671428 64.745238) (width 0.25) (layer "F.Cu") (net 8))
 (segment (start 124.671428 64.745238) (end 124.666666 64.75) (width 0.25) (layer "F.Cu") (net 8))
 (segment (start 127 76.5) (end 126.75 76.25) (width 0.25) (layer "F.Cu") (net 9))
 (segment (start 124.75 74.25) (end 124.75 68.75) (width 0.25) (layer "F.Cu") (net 9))
 (segment (start 126.75 76.25) (end 124.75 74.25) (width 0.25) (layer "F.Cu") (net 9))
 (segment (start 128 77.5) (end 126.75 76.25) (width 0.25) (layer "F.Cu") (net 9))
 (segment (start 128 82.75) (end 128 77.5) (width 0.25) (layer "F.Cu") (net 9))
 (segment (start 129 76.5) (end 127 76.5) (width 0.25) (layer "F.Cu") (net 9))
 (segment (start 137 85.25) (end 132.5 80.75) (width 0.25) (layer "F.Cu") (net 10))
 (segment (start 132.5 80.75) (end 132.5 76.5) (width 0.25) (layer "F.Cu") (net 10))
 (segment (start 132.344285 57.5) (end 132.344285 76.344285) (width 0.25) (layer "F.Cu") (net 10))
 (segment (start 132.344285 76.344285) (end 132.5 76.5) (width 0.25) (layer "F.Cu") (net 10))
 (segment (start 146.75 85.25) (end 137 85.25) (width 0.25) (layer "F.Cu") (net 10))
 (segment (start 140.017142 64.732858) (end 140 64.75) (width 0.25) (layer "F.Cu") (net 11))
 (segment (start 140.017142 57.5) (end 140.017142 64.732858) (width 0.25) (layer "F.Cu") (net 11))
 (segment (start 142 76) (end 140 74) (width 0.25) (layer "F.Cu") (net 12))
 (segment (start 142.5 76.5) (end 142 76) (width 0.25) (layer "F.Cu") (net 12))
 (segment (start 143.5 82.75) (end 143.5 77.5) (width 0.25) (layer "F.Cu") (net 12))
 (segment (start 140 74) (end 140 68.75) (width 0.25) (layer "F.Cu") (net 12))
 (segment (start 144.5 76.5) (end 142.5 76.5) (width 0.25) (layer "F.Cu") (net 12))
 (segment (start 143.5 77.5) (end 142 76) (width 0.25) (layer "F.Cu") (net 12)))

